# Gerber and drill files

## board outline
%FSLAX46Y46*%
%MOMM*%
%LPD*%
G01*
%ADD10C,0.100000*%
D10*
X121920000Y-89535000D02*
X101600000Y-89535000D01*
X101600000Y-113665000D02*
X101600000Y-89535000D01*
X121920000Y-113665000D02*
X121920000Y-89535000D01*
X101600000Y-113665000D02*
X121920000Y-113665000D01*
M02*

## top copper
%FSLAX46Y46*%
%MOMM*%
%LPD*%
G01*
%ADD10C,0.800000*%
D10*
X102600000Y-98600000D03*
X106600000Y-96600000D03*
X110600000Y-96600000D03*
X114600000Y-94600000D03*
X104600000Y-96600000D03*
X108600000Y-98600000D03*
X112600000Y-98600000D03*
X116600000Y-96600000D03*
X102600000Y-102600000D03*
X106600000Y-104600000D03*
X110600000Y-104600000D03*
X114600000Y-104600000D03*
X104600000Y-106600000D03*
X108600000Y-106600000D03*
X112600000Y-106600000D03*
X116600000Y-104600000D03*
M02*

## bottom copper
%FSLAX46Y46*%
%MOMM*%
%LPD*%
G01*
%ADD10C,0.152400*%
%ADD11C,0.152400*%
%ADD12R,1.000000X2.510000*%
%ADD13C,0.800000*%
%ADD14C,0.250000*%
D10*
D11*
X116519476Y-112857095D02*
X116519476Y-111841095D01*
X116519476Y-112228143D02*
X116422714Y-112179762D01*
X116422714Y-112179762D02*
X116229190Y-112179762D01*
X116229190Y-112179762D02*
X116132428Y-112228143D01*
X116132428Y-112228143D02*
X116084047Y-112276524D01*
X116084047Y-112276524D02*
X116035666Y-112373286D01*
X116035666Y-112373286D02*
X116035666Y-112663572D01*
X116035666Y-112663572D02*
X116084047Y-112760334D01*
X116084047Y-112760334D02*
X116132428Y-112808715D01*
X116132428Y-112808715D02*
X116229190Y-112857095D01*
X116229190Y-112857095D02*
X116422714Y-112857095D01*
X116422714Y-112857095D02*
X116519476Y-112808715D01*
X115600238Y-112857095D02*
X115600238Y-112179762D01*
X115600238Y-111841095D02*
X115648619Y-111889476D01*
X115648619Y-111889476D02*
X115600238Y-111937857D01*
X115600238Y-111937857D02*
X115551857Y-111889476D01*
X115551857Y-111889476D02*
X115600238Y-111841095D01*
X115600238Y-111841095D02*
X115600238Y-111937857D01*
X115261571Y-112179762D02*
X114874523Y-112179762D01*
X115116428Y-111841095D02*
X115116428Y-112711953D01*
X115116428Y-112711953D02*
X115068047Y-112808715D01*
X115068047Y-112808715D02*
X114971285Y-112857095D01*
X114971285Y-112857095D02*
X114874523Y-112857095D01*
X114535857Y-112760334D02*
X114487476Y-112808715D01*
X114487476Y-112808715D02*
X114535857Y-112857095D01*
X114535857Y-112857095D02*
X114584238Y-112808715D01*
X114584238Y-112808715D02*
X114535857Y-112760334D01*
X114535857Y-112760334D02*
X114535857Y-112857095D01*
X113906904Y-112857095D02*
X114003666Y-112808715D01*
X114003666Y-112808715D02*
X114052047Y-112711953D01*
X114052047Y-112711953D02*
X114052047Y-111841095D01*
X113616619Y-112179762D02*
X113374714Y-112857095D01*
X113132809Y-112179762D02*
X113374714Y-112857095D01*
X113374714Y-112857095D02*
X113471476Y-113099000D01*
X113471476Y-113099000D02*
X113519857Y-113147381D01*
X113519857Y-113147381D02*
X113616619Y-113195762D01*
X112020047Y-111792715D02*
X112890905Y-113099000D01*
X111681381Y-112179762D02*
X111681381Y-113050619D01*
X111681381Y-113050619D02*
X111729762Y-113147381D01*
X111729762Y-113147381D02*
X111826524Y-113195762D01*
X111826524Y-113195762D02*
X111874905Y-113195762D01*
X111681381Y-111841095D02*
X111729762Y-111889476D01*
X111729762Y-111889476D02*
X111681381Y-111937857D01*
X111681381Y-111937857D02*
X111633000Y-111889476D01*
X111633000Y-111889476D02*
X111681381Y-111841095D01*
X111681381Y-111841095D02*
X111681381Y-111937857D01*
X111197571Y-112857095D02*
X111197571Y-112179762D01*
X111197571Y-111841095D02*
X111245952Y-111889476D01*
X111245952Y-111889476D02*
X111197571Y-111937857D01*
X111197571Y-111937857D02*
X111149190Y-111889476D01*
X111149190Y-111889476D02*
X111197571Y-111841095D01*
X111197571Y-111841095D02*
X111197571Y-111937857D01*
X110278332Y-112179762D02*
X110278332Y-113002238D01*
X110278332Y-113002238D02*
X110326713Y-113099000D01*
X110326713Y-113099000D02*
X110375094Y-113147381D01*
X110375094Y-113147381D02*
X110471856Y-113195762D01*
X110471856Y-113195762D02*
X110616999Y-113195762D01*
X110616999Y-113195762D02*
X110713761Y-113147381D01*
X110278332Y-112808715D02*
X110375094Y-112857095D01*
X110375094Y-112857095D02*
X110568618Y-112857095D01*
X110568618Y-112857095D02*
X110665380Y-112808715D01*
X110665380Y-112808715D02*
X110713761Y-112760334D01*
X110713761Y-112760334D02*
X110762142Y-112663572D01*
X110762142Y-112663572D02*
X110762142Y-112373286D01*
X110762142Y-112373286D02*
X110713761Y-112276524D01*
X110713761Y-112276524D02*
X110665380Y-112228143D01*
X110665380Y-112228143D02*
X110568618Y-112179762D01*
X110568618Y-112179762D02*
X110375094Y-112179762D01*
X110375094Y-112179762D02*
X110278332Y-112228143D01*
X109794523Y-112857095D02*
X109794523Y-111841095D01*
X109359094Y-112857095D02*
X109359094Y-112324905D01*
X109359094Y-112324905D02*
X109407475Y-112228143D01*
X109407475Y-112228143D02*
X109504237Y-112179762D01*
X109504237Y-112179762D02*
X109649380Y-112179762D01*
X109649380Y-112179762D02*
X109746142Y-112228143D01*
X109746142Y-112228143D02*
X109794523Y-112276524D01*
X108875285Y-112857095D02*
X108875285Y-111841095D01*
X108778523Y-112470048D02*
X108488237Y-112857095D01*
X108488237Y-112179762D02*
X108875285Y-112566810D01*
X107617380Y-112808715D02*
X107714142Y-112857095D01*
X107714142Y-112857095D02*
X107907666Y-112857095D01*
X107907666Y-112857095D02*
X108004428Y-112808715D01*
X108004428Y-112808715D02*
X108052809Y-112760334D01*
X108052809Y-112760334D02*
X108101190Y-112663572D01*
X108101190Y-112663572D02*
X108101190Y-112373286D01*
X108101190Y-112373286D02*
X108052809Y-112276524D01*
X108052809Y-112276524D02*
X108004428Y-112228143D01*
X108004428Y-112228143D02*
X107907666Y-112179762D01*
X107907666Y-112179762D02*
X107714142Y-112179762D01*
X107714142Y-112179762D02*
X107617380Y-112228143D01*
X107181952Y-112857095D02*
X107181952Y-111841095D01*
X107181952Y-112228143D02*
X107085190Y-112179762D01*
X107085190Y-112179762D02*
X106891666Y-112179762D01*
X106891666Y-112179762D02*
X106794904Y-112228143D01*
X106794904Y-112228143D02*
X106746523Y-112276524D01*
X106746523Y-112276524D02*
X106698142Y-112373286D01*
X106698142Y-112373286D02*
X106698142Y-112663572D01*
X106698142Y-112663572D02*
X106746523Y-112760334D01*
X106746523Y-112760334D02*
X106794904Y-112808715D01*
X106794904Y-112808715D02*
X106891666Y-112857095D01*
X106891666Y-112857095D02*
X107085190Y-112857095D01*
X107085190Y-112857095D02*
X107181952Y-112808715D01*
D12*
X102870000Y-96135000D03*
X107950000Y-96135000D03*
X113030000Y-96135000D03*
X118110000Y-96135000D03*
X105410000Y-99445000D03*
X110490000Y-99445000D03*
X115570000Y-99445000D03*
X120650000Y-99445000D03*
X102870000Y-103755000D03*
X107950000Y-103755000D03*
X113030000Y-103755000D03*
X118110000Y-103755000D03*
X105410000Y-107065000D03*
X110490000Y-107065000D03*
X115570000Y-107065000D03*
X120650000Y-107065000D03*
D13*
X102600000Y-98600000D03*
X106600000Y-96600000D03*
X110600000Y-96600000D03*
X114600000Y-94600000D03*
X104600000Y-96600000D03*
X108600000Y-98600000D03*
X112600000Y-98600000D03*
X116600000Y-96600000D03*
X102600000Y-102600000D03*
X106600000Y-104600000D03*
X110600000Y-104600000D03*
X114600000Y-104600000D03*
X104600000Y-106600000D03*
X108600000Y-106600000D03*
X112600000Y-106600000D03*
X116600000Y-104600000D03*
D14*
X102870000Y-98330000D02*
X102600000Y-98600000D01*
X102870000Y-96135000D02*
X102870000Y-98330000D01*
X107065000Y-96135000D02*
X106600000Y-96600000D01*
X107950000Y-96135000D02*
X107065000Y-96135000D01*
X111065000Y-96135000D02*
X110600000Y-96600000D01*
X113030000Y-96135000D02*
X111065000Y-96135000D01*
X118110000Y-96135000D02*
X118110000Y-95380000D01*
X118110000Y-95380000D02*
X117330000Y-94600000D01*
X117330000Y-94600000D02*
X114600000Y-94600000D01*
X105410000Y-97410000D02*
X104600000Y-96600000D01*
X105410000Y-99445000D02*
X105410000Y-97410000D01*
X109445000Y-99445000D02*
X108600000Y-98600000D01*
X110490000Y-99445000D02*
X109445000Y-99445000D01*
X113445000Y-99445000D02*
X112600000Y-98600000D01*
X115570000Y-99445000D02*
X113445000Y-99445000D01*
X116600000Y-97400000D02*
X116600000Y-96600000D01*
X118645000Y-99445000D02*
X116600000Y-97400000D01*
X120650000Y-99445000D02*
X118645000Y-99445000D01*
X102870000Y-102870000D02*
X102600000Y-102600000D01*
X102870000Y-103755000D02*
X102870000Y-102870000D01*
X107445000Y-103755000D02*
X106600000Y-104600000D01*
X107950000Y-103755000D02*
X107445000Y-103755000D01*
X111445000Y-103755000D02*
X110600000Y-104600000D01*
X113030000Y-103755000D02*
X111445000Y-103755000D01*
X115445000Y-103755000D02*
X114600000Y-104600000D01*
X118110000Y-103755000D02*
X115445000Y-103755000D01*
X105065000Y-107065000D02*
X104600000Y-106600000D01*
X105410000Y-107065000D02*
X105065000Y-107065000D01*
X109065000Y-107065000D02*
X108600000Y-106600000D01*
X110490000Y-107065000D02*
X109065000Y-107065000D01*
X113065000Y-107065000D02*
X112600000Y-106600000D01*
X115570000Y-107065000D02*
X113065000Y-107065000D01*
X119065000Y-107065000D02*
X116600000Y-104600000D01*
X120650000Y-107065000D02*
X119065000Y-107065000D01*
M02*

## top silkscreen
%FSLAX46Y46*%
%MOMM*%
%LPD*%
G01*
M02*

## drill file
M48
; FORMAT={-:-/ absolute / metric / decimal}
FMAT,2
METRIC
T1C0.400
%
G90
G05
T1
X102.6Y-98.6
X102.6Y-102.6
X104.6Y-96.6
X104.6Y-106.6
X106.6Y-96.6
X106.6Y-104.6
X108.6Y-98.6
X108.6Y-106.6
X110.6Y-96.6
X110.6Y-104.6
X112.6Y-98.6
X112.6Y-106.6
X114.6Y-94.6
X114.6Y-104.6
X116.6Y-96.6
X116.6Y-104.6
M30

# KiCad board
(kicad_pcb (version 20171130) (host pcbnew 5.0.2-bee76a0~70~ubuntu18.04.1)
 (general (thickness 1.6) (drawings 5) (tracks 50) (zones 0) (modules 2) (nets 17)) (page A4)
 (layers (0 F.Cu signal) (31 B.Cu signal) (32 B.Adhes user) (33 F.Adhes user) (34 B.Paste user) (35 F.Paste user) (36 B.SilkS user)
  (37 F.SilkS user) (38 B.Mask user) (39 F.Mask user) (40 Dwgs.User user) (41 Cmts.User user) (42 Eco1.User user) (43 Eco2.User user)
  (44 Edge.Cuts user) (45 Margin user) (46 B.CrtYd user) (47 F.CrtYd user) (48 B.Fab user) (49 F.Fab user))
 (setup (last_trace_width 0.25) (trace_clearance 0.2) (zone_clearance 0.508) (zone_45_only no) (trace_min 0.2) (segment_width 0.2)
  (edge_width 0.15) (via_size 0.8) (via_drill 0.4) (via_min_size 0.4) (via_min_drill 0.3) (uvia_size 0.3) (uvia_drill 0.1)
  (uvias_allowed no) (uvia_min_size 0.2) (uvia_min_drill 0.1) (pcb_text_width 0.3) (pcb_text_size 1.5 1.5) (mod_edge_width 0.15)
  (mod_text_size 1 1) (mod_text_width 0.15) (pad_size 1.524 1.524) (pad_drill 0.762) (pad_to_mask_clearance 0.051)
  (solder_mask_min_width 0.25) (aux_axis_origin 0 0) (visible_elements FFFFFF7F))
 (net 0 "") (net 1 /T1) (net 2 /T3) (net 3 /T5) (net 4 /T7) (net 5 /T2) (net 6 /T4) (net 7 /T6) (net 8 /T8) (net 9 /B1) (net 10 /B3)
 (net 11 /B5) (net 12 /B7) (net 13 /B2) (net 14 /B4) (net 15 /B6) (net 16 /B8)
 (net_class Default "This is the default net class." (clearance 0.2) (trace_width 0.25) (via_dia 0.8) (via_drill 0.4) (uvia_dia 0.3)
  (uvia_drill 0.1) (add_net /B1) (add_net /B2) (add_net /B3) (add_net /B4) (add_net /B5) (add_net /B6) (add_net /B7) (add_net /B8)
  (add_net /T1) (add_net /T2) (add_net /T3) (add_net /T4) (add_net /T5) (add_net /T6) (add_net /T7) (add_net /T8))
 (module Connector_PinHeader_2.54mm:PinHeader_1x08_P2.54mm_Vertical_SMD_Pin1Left (layer B.Cu) (at 111.76 97.79 270)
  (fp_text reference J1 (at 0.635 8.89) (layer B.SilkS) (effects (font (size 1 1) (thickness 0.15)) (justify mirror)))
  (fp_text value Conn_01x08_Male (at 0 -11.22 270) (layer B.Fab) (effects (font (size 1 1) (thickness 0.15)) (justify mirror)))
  (pad 1 smd rect (at -1.655 8.89 270) (size 2.51 1) (layers B.Cu B.Paste B.Mask) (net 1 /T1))
  (pad 3 smd rect (at -1.655 3.81 270) (size 2.51 1) (layers B.Cu B.Paste B.Mask) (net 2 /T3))
  (pad 5 smd rect (at -1.655 -1.27 270) (size 2.51 1) (layers B.Cu B.Paste B.Mask) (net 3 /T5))
  (pad 7 smd rect (at -1.655 -6.35 270) (size 2.51 1) (layers B.Cu B.Paste B.Mask) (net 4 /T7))
  (pad 2 smd rect (at 1.655 6.35 270) (size 2.51 1) (layers B.Cu B.Paste B.Mask) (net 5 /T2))
  (pad 4 smd rect (at 1.655 1.27 270) (size 2.51 1) (layers B.Cu B.Paste B.Mask) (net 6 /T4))
  (pad 6 smd rect (at 1.655 -3.81 270) (size 2.51 1) (layers B.Cu B.Paste B.Mask) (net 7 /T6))
  (pad 8 smd rect (at 1.655 -8.89 270) (size 2.51 1) (layers B.Cu B.Paste B.Mask) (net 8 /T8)))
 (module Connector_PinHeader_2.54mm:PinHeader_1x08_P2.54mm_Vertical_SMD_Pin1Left (layer B.Cu) (at 111.76 105.41 270)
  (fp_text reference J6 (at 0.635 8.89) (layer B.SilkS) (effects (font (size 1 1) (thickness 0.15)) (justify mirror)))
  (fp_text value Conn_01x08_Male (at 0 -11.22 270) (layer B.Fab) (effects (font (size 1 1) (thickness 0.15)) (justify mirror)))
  (pad 1 smd rect (at -1.655 8.89 270) (size 2.51 1) (layers B.Cu B.Paste B.Mask) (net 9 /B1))
  (pad 3 smd rect (at -1.655 3.81 270) (size 2.51 1) (layers B.Cu B.Paste B.Mask) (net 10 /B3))
  (pad 5 smd rect (at -1.655 -1.27 270) (size 2.51 1) (layers B.Cu B.Paste B.Mask) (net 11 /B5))
  (pad 7 smd rect (at -1.655 -6.35 270) (size 2.51 1) (layers B.Cu B.Paste B.Mask) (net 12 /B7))
  (pad 2 smd rect (at 1.655 6.35 270) (size 2.51 1) (layers B.Cu B.Paste B.Mask) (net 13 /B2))
  (pad 4 smd rect (at 1.655 1.27 270) (size 2.51 1) (layers B.Cu B.Paste B.Mask) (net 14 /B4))
  (pad 6 smd rect (at 1.655 -3.81 270) (size 2.51 1) (layers B.Cu B.Paste B.Mask) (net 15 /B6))
  (pad 8 smd rect (at 1.655 -8.89 270) (size 2.51 1) (layers B.Cu B.Paste B.Mask) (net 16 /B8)))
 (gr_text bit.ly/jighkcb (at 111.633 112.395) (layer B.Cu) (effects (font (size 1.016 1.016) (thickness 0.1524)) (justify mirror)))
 (gr_line (start 121.92 89.535) (end 101.6 89.535) (layer Edge.Cuts) (width 0.1))
 (gr_line (start 101.6 113.665) (end 101.6 89.535) (layer Edge.Cuts) (width 0.1))
 (gr_line (start 121.92 113.665) (end 121.92 89.535) (layer Edge.Cuts) (width 0.1))
 (gr_line (start 101.6 113.665) (end 121.92 113.665) (layer Edge.Cuts) (width 0.1))
 (via (at 102.6 98.6) (size 0.8) (drill 0.4) (layers F.Cu B.Cu) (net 1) (status 1000030))
 (segment (start 102.87 98.33) (end 102.6 98.6) (width 0.25) (layer B.Cu) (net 1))
 (segment (start 102.87 96.135) (end 102.87 98.33) (width 0.25) (layer B.Cu) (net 1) (status 10))
 (via (at 106.6 96.6) (size 0.8) (drill 0.4) (layers F.Cu B.Cu) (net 2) (status 30))
 (segment (start 107.065 96.135) (end 106.6 96.6) (width 0.25) (layer B.Cu) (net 2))
 (segment (start 107.95 96.135) (end 107.065 96.135) (width 0.25) (layer B.Cu) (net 2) (status 10))
 (via (at 110.6 96.6) (size 0.8) (drill 0.4) (layers F.Cu B.Cu) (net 3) (status 30))
 (segment (start 111.065 96.135) (end 110.6 96.6) (width 0.25) (layer B.Cu) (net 3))
 (segment (start 113.03 96.135) (end 111.065 96.135) (width 0.25) (layer B.Cu) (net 3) (status 10))
 (segment (start 118.11 96.135) (end 118.11 95.38) (width 0.25) (layer B.Cu) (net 4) (status 30))
 (segment (start 118.11 95.38) (end 117.33 94.6) (width 0.25) (layer B.Cu) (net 4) (status 10))
 (via (at 114.6 94.6) (size 0.8) (drill 0.4) (layers F.Cu B.Cu) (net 4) (status 30))
 (segment (start 117.33 94.6) (end 114.6 94.6) (width 0.25) (layer B.Cu) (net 4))
 (via (at 104.6 96.6) (size 0.8) (drill 0.4) (layers F.Cu B.Cu) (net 5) (status 30))
 (segment (start 105.41 97.41) (end 104.6 96.6) (width 0.25) (layer B.Cu) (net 5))
 (segment (start 105.41 99.445) (end 105.41 97.41) (width 0.25) (layer B.Cu) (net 5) (status 10))
 (via (at 108.6 98.6) (size 0.8) (drill 0.4) (layers F.Cu B.Cu) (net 6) (status 30))
 (segment (start 109.445 99.445) (end 108.6 98.6) (width 0.25) (layer B.Cu) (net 6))
 (segment (start 110.49 99.445) (end 109.445 99.445) (width 0.25) (layer B.Cu) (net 6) (status 10))
 (via (at 112.6 98.6) (size 0.8) (drill 0.4) (layers F.Cu B.Cu) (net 7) (status 30))
 (segment (start 113.445 99.445) (end 112.6 98.6) (width 0.25) (layer B.Cu) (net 7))
 (segment (start 115.57 99.445) (end 113.445 99.445) (width 0.25) (layer B.Cu) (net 7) (status 10))
 (via (at 116.6 96.6) (size 0.8) (drill 0.4) (layers F.Cu B.Cu) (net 8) (status 30))
 (segment (start 116.6 97.4) (end 116.6 96.6) (width 0.25) (layer B.Cu) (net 8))
 (segment (start 118.645 99.445) (end 116.6 97.4) (width 0.25) (layer B.Cu) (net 8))
 (segment (start 120.65 99.445) (end 118.645 99.445) (width 0.25) (layer B.Cu) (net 8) (status 10))
 (via (at 102.6 102.6) (size 0.8) (drill 0.4) (layers F.Cu B.Cu) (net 9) (status 30))
 (segment (start 102.87 102.87) (end 102.6 102.6) (width 0.25) (layer B.Cu) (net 9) (status 30))
 (segment (start 102.87 103.755) (end 102.87 102.87) (width 0.25) (layer B.Cu) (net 9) (status 30))
 (via (at 106.6 104.6) (size 0.8) (drill 0.4) (layers F.Cu B.Cu) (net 10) (status 30))
 (segment (start 107.445 103.755) (end 106.6 104.6) (width 0.25) (layer B.Cu) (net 10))
 (segment (start 107.95 103.755) (end 107.445 103.755) (width 0.25) (layer B.Cu) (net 10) (status 10))
 (via (at 110.6 104.6) (size 0.8) (drill 0.4) (layers F.Cu B.Cu) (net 11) (status 30))
 (segment (start 111.445 103.755) (end 110.6 104.6) (width 0.25) (layer B.Cu) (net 11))
 (segment (start 113.03 103.755) (end 111.445 103.755) (width 0.25) (layer B.Cu) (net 11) (status 10))
 (via (at 114.6 104.6) (size 0.8) (drill 0.4) (layers F.Cu B.Cu) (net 12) (status 30))
 (segment (start 115.445 103.755) (end 114.6 104.6) (width 0.25) (layer B.Cu) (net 12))
 (segment (start 118.11 103.755) (end 115.445 103.755) (width 0.25) (layer B.Cu) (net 12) (status 10))
 (via (at 104.6 106.6) (size 0.8) (drill 0.4) (layers F.Cu B.Cu) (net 13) (status 30))
 (segment (start 105.065 107.065) (end 104.6 106.6) (width 0.25) (layer B.Cu) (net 13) (status 10))
 (segment (start 105.41 107.065) (end 105.065 107.065) (width 0.25) (layer B.Cu) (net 13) (status 30))
 (via (at 108.6 106.6) (size 0.8) (drill 0.4) (layers F.Cu B.Cu) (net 14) (status 1000030))
 (segment (start 109.065 107.065) (end 108.6 106.6) (width 0.25) (layer B.Cu) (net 14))
 (segment (start 110.49 107.065) (end 109.065 107.065) (width 0.25) (layer B.Cu) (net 14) (status 10))
 (via (at 112.6 106.6) (size 0.8) (drill 0.4) (layers F.Cu B.Cu) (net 15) (status 30))
 (segment (start 113.065 107.065) (end 112.6 106.6) (width 0.25) (layer B.Cu) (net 15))
 (segment (start 115.57 107.065) (end 113.065 107.065) (width 0.25) (layer B.Cu) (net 15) (status 10))
 (via (at 116.6 104.6) (size 0.8) (drill 0.4) (layers F.Cu B.Cu) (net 16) (status 30))
 (segment (start 119.065 107.065) (end 116.6 104.6) (width 0.25) (layer B.Cu) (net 16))
 (segment (start 120.65 107.065) (end 119.065 107.065) (width 0.25) (layer B.Cu) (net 16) (status 10)))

